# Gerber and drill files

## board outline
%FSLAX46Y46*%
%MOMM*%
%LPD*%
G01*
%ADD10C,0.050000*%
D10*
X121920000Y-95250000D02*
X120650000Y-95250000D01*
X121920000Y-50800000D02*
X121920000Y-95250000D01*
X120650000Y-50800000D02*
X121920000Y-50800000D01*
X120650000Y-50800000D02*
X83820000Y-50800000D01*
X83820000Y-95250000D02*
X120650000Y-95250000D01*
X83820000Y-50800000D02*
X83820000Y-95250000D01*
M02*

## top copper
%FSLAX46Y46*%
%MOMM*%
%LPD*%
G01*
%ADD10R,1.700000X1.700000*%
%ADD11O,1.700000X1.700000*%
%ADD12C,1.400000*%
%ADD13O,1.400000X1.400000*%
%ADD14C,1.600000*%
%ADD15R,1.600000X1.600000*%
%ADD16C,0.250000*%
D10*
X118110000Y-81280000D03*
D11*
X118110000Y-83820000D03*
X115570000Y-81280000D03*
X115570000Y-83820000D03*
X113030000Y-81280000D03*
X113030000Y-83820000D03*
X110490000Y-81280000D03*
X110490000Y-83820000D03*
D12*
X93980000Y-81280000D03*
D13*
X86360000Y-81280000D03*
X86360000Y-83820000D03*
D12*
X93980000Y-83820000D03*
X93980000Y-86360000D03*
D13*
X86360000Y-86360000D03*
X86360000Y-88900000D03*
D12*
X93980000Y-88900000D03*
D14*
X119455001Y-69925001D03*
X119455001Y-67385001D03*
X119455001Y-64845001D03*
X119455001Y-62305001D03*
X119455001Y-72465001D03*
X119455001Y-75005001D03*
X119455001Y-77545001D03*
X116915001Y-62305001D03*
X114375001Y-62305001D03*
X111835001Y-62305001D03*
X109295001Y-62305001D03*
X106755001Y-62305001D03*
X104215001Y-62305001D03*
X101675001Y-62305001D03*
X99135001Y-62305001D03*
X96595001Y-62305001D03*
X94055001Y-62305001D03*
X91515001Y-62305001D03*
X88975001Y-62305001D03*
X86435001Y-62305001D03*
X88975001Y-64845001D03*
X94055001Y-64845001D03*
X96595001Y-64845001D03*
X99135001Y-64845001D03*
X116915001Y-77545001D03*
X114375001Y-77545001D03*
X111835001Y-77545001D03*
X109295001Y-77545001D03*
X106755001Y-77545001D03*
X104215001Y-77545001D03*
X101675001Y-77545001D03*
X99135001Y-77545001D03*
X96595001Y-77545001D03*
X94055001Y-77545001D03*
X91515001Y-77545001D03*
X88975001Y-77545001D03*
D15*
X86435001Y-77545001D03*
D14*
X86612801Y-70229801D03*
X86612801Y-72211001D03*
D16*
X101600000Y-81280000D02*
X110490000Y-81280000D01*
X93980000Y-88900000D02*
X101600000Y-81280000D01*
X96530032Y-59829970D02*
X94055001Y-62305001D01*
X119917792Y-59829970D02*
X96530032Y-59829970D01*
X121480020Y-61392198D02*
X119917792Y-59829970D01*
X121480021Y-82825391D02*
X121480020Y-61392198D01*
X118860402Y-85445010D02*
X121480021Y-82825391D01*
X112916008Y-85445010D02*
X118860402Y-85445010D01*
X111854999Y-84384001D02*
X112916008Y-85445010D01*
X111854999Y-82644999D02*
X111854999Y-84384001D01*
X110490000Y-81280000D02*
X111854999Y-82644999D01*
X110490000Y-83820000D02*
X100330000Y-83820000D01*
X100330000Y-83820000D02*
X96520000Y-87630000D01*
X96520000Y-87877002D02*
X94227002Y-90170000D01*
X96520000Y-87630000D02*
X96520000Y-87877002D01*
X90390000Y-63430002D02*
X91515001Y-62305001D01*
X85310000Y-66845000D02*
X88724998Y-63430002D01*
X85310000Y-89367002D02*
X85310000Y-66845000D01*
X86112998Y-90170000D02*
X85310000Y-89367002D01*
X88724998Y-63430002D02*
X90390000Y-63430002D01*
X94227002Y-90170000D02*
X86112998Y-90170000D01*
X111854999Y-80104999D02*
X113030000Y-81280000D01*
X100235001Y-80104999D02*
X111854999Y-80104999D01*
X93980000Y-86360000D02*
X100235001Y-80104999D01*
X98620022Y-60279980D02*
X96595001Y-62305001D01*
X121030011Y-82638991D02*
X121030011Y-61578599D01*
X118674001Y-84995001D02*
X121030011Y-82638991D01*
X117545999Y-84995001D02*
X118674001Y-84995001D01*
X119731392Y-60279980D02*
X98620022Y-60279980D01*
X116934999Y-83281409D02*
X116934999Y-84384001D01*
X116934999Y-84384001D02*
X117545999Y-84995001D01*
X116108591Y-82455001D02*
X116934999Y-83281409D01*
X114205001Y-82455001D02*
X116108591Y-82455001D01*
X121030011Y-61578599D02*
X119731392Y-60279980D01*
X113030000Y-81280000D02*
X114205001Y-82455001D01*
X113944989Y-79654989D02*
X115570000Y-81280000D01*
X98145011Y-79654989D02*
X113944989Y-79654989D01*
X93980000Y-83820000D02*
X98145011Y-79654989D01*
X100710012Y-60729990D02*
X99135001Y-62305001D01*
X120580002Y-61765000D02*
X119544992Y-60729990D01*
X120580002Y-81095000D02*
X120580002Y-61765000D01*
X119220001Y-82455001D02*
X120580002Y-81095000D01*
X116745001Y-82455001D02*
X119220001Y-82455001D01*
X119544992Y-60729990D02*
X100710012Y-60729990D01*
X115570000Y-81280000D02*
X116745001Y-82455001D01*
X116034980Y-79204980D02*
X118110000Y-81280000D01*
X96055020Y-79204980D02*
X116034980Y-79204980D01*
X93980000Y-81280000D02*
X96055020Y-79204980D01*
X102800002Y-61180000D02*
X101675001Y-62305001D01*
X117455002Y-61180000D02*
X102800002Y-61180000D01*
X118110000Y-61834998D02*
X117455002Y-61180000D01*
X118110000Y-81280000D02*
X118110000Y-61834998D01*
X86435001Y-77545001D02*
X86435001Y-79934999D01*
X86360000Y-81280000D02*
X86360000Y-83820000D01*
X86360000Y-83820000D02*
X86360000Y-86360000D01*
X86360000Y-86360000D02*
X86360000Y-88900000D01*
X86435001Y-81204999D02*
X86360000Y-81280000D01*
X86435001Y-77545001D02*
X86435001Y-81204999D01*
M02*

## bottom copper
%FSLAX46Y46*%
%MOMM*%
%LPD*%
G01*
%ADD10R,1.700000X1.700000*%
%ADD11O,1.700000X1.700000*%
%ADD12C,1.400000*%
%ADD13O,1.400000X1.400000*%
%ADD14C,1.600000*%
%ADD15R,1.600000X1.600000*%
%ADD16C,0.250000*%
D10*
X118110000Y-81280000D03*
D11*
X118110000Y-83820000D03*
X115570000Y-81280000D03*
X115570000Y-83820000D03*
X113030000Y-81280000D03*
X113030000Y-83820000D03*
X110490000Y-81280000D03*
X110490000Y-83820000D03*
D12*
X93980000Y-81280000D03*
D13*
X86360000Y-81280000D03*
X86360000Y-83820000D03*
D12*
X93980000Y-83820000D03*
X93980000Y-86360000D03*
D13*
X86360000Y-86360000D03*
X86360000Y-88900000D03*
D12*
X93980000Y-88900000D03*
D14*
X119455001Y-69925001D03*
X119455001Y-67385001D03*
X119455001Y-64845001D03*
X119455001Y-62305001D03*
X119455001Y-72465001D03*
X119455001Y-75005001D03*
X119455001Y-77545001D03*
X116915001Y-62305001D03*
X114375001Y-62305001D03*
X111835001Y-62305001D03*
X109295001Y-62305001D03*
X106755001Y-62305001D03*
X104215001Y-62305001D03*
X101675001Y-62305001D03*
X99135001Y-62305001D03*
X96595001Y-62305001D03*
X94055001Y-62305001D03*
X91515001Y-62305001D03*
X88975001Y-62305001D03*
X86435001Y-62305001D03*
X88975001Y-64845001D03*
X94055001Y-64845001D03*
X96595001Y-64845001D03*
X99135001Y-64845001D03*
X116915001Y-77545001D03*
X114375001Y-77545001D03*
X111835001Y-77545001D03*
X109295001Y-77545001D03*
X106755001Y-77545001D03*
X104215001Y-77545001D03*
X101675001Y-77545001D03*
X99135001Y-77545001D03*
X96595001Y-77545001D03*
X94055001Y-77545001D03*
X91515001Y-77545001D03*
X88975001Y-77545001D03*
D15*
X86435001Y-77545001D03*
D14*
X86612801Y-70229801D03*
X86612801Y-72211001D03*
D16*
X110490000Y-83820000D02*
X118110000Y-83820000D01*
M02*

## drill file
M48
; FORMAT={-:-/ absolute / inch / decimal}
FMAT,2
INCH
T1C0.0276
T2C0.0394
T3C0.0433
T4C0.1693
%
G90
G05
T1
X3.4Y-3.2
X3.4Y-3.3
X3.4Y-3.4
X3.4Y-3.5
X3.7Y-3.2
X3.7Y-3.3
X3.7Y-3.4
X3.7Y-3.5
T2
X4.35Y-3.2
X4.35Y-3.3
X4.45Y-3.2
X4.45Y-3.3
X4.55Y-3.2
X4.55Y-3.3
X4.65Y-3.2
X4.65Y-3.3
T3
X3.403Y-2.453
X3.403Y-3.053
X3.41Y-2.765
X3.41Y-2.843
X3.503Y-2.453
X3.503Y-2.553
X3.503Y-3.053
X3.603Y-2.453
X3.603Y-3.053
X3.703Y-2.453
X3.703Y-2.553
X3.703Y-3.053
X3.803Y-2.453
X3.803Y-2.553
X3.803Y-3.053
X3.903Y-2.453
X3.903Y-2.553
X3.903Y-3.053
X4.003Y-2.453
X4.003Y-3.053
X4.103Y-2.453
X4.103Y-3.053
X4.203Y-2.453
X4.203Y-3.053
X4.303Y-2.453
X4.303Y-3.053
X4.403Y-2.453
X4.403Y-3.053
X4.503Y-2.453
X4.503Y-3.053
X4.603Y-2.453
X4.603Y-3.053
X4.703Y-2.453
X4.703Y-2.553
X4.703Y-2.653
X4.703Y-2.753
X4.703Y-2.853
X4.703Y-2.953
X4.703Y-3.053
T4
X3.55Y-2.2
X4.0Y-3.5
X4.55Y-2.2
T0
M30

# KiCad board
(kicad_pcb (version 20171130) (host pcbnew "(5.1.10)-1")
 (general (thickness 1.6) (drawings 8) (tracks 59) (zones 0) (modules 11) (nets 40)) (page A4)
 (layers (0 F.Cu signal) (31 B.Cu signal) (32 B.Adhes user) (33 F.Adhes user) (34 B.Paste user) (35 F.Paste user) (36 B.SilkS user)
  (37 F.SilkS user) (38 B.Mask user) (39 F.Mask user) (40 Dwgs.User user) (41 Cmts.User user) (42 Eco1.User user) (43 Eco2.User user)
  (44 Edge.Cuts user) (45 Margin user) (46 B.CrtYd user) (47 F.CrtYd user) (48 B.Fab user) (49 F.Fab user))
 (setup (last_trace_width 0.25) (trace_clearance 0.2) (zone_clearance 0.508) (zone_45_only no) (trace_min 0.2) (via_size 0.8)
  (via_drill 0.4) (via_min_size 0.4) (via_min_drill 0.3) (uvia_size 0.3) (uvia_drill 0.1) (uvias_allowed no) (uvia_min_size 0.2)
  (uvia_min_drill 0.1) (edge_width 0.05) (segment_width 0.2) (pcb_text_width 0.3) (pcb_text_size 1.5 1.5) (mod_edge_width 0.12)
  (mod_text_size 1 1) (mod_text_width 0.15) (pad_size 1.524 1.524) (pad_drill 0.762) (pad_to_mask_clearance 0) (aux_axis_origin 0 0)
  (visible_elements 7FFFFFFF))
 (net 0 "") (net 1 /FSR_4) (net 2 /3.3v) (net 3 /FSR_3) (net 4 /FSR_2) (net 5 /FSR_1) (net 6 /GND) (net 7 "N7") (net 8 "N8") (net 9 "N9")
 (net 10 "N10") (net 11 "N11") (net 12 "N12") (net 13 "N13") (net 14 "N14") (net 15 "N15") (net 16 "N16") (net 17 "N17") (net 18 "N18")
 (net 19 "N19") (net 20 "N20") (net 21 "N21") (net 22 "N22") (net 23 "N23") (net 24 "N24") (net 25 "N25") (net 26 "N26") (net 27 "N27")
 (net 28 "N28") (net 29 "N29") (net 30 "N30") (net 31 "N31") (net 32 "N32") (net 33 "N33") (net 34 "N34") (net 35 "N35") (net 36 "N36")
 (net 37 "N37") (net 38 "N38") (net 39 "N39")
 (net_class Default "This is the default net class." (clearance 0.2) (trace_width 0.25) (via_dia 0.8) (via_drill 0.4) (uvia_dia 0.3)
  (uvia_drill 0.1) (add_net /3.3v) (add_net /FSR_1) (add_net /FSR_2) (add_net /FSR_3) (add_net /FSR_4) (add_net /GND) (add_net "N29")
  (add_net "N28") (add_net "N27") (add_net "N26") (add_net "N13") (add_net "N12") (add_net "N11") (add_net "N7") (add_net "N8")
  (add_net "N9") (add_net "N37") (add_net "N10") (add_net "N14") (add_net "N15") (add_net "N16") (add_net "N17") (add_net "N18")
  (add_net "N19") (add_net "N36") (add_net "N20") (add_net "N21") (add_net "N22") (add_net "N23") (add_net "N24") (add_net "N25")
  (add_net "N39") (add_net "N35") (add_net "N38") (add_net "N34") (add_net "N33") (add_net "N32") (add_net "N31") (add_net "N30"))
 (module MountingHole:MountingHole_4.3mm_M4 (layer F.Cu) (at 101.6 88.9)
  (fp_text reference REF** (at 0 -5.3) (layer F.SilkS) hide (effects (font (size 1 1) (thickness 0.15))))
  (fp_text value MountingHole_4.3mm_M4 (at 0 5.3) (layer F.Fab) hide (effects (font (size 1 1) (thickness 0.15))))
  (pad 1 np_thru_hole circle (at 0 0) (size 4.3 4.3) (drill 4.3) (layers *.Cu *.Mask)))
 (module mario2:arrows (layer F.Cu) (at 102.87 55.88)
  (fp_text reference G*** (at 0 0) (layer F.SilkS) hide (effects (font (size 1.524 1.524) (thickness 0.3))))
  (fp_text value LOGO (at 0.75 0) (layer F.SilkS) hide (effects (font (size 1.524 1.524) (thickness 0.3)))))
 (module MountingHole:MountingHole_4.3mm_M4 (layer F.Cu) (at 115.57 55.88)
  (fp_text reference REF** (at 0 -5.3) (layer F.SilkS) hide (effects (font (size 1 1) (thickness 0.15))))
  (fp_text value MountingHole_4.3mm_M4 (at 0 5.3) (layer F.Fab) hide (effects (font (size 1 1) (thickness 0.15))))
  (pad 1 np_thru_hole circle (at 0 0) (size 4.3 4.3) (drill 4.3) (layers *.Cu *.Mask)))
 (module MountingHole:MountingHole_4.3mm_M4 (layer F.Cu) (at 90.17 55.88)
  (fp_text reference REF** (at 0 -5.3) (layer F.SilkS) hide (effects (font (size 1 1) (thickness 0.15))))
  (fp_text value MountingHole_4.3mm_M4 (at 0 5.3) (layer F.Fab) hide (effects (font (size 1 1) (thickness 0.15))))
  (pad 1 np_thru_hole circle (at 0 0) (size 4.3 4.3) (drill 4.3) (layers *.Cu *.Mask)))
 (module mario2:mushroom (layer F.Cu) (at 101.6 81.28)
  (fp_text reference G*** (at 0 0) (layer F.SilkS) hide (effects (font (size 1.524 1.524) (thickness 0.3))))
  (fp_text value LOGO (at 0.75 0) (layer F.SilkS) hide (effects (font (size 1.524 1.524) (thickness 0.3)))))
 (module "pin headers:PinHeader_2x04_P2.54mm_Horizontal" (layer F.Cu) (at 118.11 81.28 270)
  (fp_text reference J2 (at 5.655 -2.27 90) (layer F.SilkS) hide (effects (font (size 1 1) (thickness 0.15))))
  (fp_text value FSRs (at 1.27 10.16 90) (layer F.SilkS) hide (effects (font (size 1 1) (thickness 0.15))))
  (pad 1 thru_hole rect (at 0 0 270) (size 1.7 1.7) (drill 1) (layers *.Cu *.Mask) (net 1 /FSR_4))
  (pad 2 thru_hole oval (at 2.54 0 270) (size 1.7 1.7) (drill 1) (layers *.Cu *.Mask) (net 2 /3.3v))
  (pad 3 thru_hole oval (at 0 2.54 270) (size 1.7 1.7) (drill 1) (layers *.Cu *.Mask) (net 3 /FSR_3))
  (pad 4 thru_hole oval (at 2.54 2.54 270) (size 1.7 1.7) (drill 1) (layers *.Cu *.Mask) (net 2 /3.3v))
  (pad 5 thru_hole oval (at 0 5.08 270) (size 1.7 1.7) (drill 1) (layers *.Cu *.Mask) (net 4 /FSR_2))
  (pad 6 thru_hole oval (at 2.54 5.08 270) (size 1.7 1.7) (drill 1) (layers *.Cu *.Mask) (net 2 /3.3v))
  (pad 7 thru_hole oval (at 0 7.62 270) (size 1.7 1.7) (drill 1) (layers *.Cu *.Mask) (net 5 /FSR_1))
  (pad 8 thru_hole oval (at 2.54 7.62 270) (size 1.7 1.7) (drill 1) (layers *.Cu *.Mask) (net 2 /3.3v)))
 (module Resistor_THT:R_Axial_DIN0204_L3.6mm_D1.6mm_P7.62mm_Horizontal (layer F.Cu) (at 93.98 81.28 180)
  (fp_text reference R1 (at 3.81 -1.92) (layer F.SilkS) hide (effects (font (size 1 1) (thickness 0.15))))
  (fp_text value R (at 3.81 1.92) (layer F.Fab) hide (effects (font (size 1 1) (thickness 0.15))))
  (pad 1 thru_hole circle (at 0 0 180) (size 1.4 1.4) (drill 0.7) (layers *.Cu *.Mask) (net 1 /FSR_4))
  (pad 2 thru_hole oval (at 7.62 0 180) (size 1.4 1.4) (drill 0.7) (layers *.Cu *.Mask) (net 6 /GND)))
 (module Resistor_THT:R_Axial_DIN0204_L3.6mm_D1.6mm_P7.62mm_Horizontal (layer F.Cu) (at 93.98 83.82 180)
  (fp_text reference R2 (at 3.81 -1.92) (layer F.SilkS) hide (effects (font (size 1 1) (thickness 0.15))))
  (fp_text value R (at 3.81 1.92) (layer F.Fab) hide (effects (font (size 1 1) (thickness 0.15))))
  (pad 2 thru_hole oval (at 7.62 0 180) (size 1.4 1.4) (drill 0.7) (layers *.Cu *.Mask) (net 6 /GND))
  (pad 1 thru_hole circle (at 0 0 180) (size 1.4 1.4) (drill 0.7) (layers *.Cu *.Mask) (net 3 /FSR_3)))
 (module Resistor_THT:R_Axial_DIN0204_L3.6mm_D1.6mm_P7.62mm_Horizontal (layer F.Cu) (at 93.98 86.36 180)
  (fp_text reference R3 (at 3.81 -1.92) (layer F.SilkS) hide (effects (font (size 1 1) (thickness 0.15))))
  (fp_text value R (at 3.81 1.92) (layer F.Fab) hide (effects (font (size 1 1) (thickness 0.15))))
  (pad 1 thru_hole circle (at 0 0 180) (size 1.4 1.4) (drill 0.7) (layers *.Cu *.Mask) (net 4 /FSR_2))
  (pad 2 thru_hole oval (at 7.62 0 180) (size 1.4 1.4) (drill 0.7) (layers *.Cu *.Mask) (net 6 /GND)))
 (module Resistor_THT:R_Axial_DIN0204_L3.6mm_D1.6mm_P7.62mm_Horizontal (layer F.Cu) (at 93.98 88.9 180)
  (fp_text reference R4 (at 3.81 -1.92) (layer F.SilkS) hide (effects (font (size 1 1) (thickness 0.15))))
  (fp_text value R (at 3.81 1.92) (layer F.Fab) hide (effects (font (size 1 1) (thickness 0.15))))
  (pad 2 thru_hole oval (at 7.62 0 180) (size 1.4 1.4) (drill 0.7) (layers *.Cu *.Mask) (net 6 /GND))
  (pad 1 thru_hole circle (at 0 0 180) (size 1.4 1.4) (drill 0.7) (layers *.Cu *.Mask) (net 5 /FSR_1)))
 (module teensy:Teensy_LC (layer F.Cu) (at 102.945001 69.925001)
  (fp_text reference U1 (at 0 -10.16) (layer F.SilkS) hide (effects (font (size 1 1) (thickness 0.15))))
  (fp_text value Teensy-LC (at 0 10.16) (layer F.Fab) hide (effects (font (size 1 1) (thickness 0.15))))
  (pad 17 thru_hole circle (at 16.51 0) (size 1.6 1.6) (drill 1.1) (layers *.Cu *.Mask) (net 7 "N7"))
  (pad 18 thru_hole circle (at 16.51 -2.54) (size 1.6 1.6) (drill 1.1) (layers *.Cu *.Mask) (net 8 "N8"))
  (pad 19 thru_hole circle (at 16.51 -5.08) (size 1.6 1.6) (drill 1.1) (layers *.Cu *.Mask) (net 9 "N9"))
  (pad 20 thru_hole circle (at 16.51 -7.62) (size 1.6 1.6) (drill 1.1) (layers *.Cu *.Mask) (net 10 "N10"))
  (pad 16 thru_hole circle (at 16.51 2.54) (size 1.6 1.6) (drill 1.1) (layers *.Cu *.Mask) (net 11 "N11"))
  (pad 15 thru_hole circle (at 16.51 5.08) (size 1.6 1.6) (drill 1.1) (layers *.Cu *.Mask) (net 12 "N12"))
  (pad 14 thru_hole circle (at 16.51 7.62) (size 1.6 1.6) (drill 1.1) (layers *.Cu *.Mask) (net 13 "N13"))
  (pad 21 thru_hole circle (at 13.97 -7.62) (size 1.6 1.6) (drill 1.1) (layers *.Cu *.Mask) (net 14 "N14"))
  (pad 22 thru_hole circle (at 11.43 -7.62) (size 1.6 1.6) (drill 1.1) (layers *.Cu *.Mask) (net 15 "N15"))
  (pad 23 thru_hole circle (at 8.89 -7.62) (size 1.6 1.6) (drill 1.1) (layers *.Cu *.Mask) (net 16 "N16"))
  (pad 24 thru_hole circle (at 6.35 -7.62) (size 1.6 1.6) (drill 1.1) (layers *.Cu *.Mask) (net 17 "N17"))
  (pad 25 thru_hole circle (at 3.81 -7.62) (size 1.6 1.6) (drill 1.1) (layers *.Cu *.Mask) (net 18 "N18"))
  (pad 26 thru_hole circle (at 1.27 -7.62) (size 1.6 1.6) (drill 1.1) (layers *.Cu *.Mask) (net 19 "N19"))
  (pad 27 thru_hole circle (at -1.27 -7.62) (size 1.6 1.6) (drill 1.1) (layers *.Cu *.Mask) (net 1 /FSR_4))
  (pad 28 thru_hole circle (at -3.81 -7.62) (size 1.6 1.6) (drill 1.1) (layers *.Cu *.Mask) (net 3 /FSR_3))
  (pad 29 thru_hole circle (at -6.35 -7.62) (size 1.6 1.6) (drill 1.1) (layers *.Cu *.Mask) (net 4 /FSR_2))
  (pad 30 thru_hole circle (at -8.89 -7.62) (size 1.6 1.6) (drill 1.1) (layers *.Cu *.Mask) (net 5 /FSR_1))
  (pad 31 thru_hole circle (at -11.43 -7.62) (size 1.6 1.6) (drill 1.1) (layers *.Cu *.Mask) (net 2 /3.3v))
  (pad 32 thru_hole circle (at -13.97 -7.62) (size 1.6 1.6) (drill 1.1) (layers *.Cu *.Mask) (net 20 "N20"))
  (pad 33 thru_hole circle (at -16.51 -7.62) (size 1.6 1.6) (drill 1.1) (layers *.Cu *.Mask) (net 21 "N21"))
  (pad 34 thru_hole circle (at -13.97 -5.08) (size 1.6 1.6) (drill 1.1) (layers *.Cu *.Mask) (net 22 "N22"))
  (pad 35 thru_hole circle (at -8.89 -5.08) (size 1.6 1.6) (drill 1.1) (layers *.Cu *.Mask) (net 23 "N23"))
  (pad 36 thru_hole circle (at -6.35 -5.08) (size 1.6 1.6) (drill 1.1) (layers *.Cu *.Mask) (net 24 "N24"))
  (pad 37 thru_hole circle (at -3.81 -5.08) (size 1.6 1.6) (drill 1.1) (layers *.Cu *.Mask) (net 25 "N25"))
  (pad 13 thru_hole circle (at 13.97 7.62) (size 1.6 1.6) (drill 1.1) (layers *.Cu *.Mask) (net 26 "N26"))
  (pad 12 thru_hole circle (at 11.43 7.62) (size 1.6 1.6) (drill 1.1) (layers *.Cu *.Mask) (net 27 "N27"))
  (pad 11 thru_hole circle (at 8.89 7.62) (size 1.6 1.6) (drill 1.1) (layers *.Cu *.Mask) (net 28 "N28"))
  (pad 10 thru_hole circle (at 6.35 7.62) (size 1.6 1.6) (drill 1.1) (layers *.Cu *.Mask) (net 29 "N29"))
  (pad 9 thru_hole circle (at 3.81 7.62) (size 1.6 1.6) (drill 1.1) (layers *.Cu *.Mask) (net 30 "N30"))
  (pad 8 thru_hole circle (at 1.27 7.62) (size 1.6 1.6) (drill 1.1) (layers *.Cu *.Mask) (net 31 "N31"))
  (pad 7 thru_hole circle (at -1.27 7.62) (size 1.6 1.6) (drill 1.1) (layers *.Cu *.Mask) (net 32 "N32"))
  (pad 6 thru_hole circle (at -3.81 7.62) (size 1.6 1.6) (drill 1.1) (layers *.Cu *.Mask) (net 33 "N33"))
  (pad 5 thru_hole circle (at -6.35 7.62) (size 1.6 1.6) (drill 1.1) (layers *.Cu *.Mask) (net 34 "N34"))
  (pad 4 thru_hole circle (at -8.89 7.62) (size 1.6 1.6) (drill 1.1) (layers *.Cu *.Mask) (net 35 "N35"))
  (pad 3 thru_hole circle (at -11.43 7.62) (size 1.6 1.6) (drill 1.1) (layers *.Cu *.Mask) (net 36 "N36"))
  (pad 2 thru_hole circle (at -13.97 7.62) (size 1.6 1.6) (drill 1.1) (layers *.Cu *.Mask) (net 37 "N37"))
  (pad 1 thru_hole rect (at -16.51 7.62) (size 1.6 1.6) (drill 1.1) (layers *.Cu *.Mask) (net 6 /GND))
  (pad 40 thru_hole circle (at -16.3322 0.3048) (size 1.6 1.6) (drill 1.1) (layers *.Cu *.Mask) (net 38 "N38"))
  (pad 39 thru_hole circle (at -16.3322 2.286) (size 1.6 1.6) (drill 1.1) (layers *.Cu *.Mask) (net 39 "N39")))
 (gr_line (start 121.92 95.25) (end 120.65 95.25) (layer Edge.Cuts) (width 0.05))
 (gr_line (start 121.92 50.8) (end 121.92 95.25) (layer Edge.Cuts) (width 0.05))
 (gr_line (start 120.65 50.8) (end 121.92 50.8) (layer Edge.Cuts) (width 0.05))
 (gr_line (start 120.65 50.8) (end 83.82 50.8) (layer Edge.Cuts) (width 0.05))
 (gr_line (start 83.82 95.25) (end 120.65 95.25) (layer Edge.Cuts) (width 0.05))
 (gr_line (start 83.82 50.8) (end 83.82 95.25) (layer Edge.Cuts) (width 0.05))
 (segment (start 101.6 81.28) (end 110.49 81.28) (width 0.25) (layer F.Cu) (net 5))
 (segment (start 93.98 88.9) (end 101.6 81.28) (width 0.25) (layer F.Cu) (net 5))
 (segment (start 96.530032 59.82997) (end 94.055001 62.305001) (width 0.25) (layer F.Cu) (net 5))
 (segment (start 119.917792 59.82997) (end 96.530032 59.82997) (width 0.25) (layer F.Cu) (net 5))
 (segment (start 121.48002 61.392198) (end 119.917792 59.82997) (width 0.25) (layer F.Cu) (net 5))
 (segment (start 121.480021 82.825391) (end 121.48002 61.392198) (width 0.25) (layer F.Cu) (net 5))
 (segment (start 118.860402 85.44501) (end 121.480021 82.825391) (width 0.25) (layer F.Cu) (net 5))
 (segment (start 112.916008 85.44501) (end 118.860402 85.44501) (width 0.25) (layer F.Cu) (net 5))
 (segment (start 111.854999 84.384001) (end 112.916008 85.44501) (width 0.25) (layer F.Cu) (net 5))
 (segment (start 111.854999 82.644999) (end 111.854999 84.384001) (width 0.25) (layer F.Cu) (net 5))
 (segment (start 110.49 81.28) (end 111.854999 82.644999) (width 0.25) (layer F.Cu) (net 5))
 (segment (start 110.49 83.82) (end 100.33 83.82) (width 0.25) (layer F.Cu) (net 2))
 (segment (start 100.33 83.82) (end 96.52 87.63) (width 0.25) (layer F.Cu) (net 2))
 (segment (start 96.52 87.877002) (end 94.227002 90.17) (width 0.25) (layer F.Cu) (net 2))
 (segment (start 96.52 87.63) (end 96.52 87.877002) (width 0.25) (layer F.Cu) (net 2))
 (segment (start 90.39 63.430002) (end 91.515001 62.305001) (width 0.25) (layer F.Cu) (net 2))
 (segment (start 85.31 66.845) (end 88.724998 63.430002) (width 0.25) (layer F.Cu) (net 2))
 (segment (start 85.31 89.367002) (end 85.31 66.845) (width 0.25) (layer F.Cu) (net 2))
 (segment (start 86.112998 90.17) (end 85.31 89.367002) (width 0.25) (layer F.Cu) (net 2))
 (segment (start 88.724998 63.430002) (end 90.39 63.430002) (width 0.25) (layer F.Cu) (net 2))
 (segment (start 94.227002 90.17) (end 86.112998 90.17) (width 0.25) (layer F.Cu) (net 2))
 (segment (start 110.49 83.82) (end 118.11 83.82) (width 0.25) (layer B.Cu) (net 2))
 (segment (start 111.854999 80.104999) (end 113.03 81.28) (width 0.25) (layer F.Cu) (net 4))
 (segment (start 100.235001 80.104999) (end 111.854999 80.104999) (width 0.25) (layer F.Cu) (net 4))
 (segment (start 93.98 86.36) (end 100.235001 80.104999) (width 0.25) (layer F.Cu) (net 4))
 (segment (start 98.620022 60.27998) (end 96.595001 62.305001) (width 0.25) (layer F.Cu) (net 4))
 (segment (start 121.030011 82.638991) (end 121.030011 61.578599) (width 0.25) (layer F.Cu) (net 4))
 (segment (start 118.674001 84.995001) (end 121.030011 82.638991) (width 0.25) (layer F.Cu) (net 4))
 (segment (start 117.545999 84.995001) (end 118.674001 84.995001) (width 0.25) (layer F.Cu) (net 4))
 (segment (start 119.731392 60.27998) (end 98.620022 60.27998) (width 0.25) (layer F.Cu) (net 4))
 (segment (start 116.934999 83.281409) (end 116.934999 84.384001) (width 0.25) (layer F.Cu) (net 4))
 (segment (start 116.934999 84.384001) (end 117.545999 84.995001) (width 0.25) (layer F.Cu) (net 4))
 (segment (start 116.108591 82.455001) (end 116.934999 83.281409) (width 0.25) (layer F.Cu) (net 4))
 (segment (start 114.205001 82.455001) (end 116.108591 82.455001) (width 0.25) (layer F.Cu) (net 4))
 (segment (start 121.030011 61.578599) (end 119.731392 60.27998) (width 0.25) (layer F.Cu) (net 4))
 (segment (start 113.03 81.28) (end 114.205001 82.455001) (width 0.25) (layer F.Cu) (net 4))
 (segment (start 113.944989 79.654989) (end 115.57 81.28) (width 0.25) (layer F.Cu) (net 3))
 (segment (start 98.145011 79.654989) (end 113.944989 79.654989) (width 0.25) (layer F.Cu) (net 3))
 (segment (start 93.98 83.82) (end 98.145011 79.654989) (width 0.25) (layer F.Cu) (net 3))
 (segment (start 100.710012 60.72999) (end 99.135001 62.305001) (width 0.25) (layer F.Cu) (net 3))
 (segment (start 120.580002 61.765) (end 119.544992 60.72999) (width 0.25) (layer F.Cu) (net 3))
 (segment (start 120.580002 81.095) (end 120.580002 61.765) (width 0.25) (layer F.Cu) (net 3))
 (segment (start 119.220001 82.455001) (end 120.580002 81.095) (width 0.25) (layer F.Cu) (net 3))
 (segment (start 116.745001 82.455001) (end 119.220001 82.455001) (width 0.25) (layer F.Cu) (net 3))
 (segment (start 119.544992 60.72999) (end 100.710012 60.72999) (width 0.25) (layer F.Cu) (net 3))
 (segment (start 115.57 81.28) (end 116.745001 82.455001) (width 0.25) (layer F.Cu) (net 3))
 (segment (start 116.03498 79.20498) (end 118.11 81.28) (width 0.25) (layer F.Cu) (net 1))
 (segment (start 96.05502 79.20498) (end 116.03498 79.20498) (width 0.25) (layer F.Cu) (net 1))
 (segment (start 93.98 81.28) (end 96.05502 79.20498) (width 0.25) (layer F.Cu) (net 1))
 (segment (start 102.800002 61.18) (end 101.675001 62.305001) (width 0.25) (layer F.Cu) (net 1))
 (segment (start 117.455002 61.18) (end 102.800002 61.18) (width 0.25) (layer F.Cu) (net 1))
 (segment (start 118.11 61.834998) (end 117.455002 61.18) (width 0.25) (layer F.Cu) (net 1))
 (segment (start 118.11 81.28) (end 118.11 61.834998) (width 0.25) (layer F.Cu) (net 1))
 (segment (start 86.435001 77.545001) (end 86.435001 79.934999) (width 0.25) (layer F.Cu) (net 6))
 (segment (start 86.36 81.28) (end 86.36 83.82) (width 0.25) (layer F.Cu) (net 6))
 (segment (start 86.36 83.82) (end 86.36 86.36) (width 0.25) (layer F.Cu) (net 6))
 (segment (start 86.36 86.36) (end 86.36 88.9) (width 0.25) (layer F.Cu) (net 6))
 (segment (start 86.435001 81.204999) (end 86.36 81.28) (width 0.25) (layer F.Cu) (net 6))
 (segment (start 86.435001 77.545001) (end 86.435001 81.204999) (width 0.25) (layer F.Cu) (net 6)))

